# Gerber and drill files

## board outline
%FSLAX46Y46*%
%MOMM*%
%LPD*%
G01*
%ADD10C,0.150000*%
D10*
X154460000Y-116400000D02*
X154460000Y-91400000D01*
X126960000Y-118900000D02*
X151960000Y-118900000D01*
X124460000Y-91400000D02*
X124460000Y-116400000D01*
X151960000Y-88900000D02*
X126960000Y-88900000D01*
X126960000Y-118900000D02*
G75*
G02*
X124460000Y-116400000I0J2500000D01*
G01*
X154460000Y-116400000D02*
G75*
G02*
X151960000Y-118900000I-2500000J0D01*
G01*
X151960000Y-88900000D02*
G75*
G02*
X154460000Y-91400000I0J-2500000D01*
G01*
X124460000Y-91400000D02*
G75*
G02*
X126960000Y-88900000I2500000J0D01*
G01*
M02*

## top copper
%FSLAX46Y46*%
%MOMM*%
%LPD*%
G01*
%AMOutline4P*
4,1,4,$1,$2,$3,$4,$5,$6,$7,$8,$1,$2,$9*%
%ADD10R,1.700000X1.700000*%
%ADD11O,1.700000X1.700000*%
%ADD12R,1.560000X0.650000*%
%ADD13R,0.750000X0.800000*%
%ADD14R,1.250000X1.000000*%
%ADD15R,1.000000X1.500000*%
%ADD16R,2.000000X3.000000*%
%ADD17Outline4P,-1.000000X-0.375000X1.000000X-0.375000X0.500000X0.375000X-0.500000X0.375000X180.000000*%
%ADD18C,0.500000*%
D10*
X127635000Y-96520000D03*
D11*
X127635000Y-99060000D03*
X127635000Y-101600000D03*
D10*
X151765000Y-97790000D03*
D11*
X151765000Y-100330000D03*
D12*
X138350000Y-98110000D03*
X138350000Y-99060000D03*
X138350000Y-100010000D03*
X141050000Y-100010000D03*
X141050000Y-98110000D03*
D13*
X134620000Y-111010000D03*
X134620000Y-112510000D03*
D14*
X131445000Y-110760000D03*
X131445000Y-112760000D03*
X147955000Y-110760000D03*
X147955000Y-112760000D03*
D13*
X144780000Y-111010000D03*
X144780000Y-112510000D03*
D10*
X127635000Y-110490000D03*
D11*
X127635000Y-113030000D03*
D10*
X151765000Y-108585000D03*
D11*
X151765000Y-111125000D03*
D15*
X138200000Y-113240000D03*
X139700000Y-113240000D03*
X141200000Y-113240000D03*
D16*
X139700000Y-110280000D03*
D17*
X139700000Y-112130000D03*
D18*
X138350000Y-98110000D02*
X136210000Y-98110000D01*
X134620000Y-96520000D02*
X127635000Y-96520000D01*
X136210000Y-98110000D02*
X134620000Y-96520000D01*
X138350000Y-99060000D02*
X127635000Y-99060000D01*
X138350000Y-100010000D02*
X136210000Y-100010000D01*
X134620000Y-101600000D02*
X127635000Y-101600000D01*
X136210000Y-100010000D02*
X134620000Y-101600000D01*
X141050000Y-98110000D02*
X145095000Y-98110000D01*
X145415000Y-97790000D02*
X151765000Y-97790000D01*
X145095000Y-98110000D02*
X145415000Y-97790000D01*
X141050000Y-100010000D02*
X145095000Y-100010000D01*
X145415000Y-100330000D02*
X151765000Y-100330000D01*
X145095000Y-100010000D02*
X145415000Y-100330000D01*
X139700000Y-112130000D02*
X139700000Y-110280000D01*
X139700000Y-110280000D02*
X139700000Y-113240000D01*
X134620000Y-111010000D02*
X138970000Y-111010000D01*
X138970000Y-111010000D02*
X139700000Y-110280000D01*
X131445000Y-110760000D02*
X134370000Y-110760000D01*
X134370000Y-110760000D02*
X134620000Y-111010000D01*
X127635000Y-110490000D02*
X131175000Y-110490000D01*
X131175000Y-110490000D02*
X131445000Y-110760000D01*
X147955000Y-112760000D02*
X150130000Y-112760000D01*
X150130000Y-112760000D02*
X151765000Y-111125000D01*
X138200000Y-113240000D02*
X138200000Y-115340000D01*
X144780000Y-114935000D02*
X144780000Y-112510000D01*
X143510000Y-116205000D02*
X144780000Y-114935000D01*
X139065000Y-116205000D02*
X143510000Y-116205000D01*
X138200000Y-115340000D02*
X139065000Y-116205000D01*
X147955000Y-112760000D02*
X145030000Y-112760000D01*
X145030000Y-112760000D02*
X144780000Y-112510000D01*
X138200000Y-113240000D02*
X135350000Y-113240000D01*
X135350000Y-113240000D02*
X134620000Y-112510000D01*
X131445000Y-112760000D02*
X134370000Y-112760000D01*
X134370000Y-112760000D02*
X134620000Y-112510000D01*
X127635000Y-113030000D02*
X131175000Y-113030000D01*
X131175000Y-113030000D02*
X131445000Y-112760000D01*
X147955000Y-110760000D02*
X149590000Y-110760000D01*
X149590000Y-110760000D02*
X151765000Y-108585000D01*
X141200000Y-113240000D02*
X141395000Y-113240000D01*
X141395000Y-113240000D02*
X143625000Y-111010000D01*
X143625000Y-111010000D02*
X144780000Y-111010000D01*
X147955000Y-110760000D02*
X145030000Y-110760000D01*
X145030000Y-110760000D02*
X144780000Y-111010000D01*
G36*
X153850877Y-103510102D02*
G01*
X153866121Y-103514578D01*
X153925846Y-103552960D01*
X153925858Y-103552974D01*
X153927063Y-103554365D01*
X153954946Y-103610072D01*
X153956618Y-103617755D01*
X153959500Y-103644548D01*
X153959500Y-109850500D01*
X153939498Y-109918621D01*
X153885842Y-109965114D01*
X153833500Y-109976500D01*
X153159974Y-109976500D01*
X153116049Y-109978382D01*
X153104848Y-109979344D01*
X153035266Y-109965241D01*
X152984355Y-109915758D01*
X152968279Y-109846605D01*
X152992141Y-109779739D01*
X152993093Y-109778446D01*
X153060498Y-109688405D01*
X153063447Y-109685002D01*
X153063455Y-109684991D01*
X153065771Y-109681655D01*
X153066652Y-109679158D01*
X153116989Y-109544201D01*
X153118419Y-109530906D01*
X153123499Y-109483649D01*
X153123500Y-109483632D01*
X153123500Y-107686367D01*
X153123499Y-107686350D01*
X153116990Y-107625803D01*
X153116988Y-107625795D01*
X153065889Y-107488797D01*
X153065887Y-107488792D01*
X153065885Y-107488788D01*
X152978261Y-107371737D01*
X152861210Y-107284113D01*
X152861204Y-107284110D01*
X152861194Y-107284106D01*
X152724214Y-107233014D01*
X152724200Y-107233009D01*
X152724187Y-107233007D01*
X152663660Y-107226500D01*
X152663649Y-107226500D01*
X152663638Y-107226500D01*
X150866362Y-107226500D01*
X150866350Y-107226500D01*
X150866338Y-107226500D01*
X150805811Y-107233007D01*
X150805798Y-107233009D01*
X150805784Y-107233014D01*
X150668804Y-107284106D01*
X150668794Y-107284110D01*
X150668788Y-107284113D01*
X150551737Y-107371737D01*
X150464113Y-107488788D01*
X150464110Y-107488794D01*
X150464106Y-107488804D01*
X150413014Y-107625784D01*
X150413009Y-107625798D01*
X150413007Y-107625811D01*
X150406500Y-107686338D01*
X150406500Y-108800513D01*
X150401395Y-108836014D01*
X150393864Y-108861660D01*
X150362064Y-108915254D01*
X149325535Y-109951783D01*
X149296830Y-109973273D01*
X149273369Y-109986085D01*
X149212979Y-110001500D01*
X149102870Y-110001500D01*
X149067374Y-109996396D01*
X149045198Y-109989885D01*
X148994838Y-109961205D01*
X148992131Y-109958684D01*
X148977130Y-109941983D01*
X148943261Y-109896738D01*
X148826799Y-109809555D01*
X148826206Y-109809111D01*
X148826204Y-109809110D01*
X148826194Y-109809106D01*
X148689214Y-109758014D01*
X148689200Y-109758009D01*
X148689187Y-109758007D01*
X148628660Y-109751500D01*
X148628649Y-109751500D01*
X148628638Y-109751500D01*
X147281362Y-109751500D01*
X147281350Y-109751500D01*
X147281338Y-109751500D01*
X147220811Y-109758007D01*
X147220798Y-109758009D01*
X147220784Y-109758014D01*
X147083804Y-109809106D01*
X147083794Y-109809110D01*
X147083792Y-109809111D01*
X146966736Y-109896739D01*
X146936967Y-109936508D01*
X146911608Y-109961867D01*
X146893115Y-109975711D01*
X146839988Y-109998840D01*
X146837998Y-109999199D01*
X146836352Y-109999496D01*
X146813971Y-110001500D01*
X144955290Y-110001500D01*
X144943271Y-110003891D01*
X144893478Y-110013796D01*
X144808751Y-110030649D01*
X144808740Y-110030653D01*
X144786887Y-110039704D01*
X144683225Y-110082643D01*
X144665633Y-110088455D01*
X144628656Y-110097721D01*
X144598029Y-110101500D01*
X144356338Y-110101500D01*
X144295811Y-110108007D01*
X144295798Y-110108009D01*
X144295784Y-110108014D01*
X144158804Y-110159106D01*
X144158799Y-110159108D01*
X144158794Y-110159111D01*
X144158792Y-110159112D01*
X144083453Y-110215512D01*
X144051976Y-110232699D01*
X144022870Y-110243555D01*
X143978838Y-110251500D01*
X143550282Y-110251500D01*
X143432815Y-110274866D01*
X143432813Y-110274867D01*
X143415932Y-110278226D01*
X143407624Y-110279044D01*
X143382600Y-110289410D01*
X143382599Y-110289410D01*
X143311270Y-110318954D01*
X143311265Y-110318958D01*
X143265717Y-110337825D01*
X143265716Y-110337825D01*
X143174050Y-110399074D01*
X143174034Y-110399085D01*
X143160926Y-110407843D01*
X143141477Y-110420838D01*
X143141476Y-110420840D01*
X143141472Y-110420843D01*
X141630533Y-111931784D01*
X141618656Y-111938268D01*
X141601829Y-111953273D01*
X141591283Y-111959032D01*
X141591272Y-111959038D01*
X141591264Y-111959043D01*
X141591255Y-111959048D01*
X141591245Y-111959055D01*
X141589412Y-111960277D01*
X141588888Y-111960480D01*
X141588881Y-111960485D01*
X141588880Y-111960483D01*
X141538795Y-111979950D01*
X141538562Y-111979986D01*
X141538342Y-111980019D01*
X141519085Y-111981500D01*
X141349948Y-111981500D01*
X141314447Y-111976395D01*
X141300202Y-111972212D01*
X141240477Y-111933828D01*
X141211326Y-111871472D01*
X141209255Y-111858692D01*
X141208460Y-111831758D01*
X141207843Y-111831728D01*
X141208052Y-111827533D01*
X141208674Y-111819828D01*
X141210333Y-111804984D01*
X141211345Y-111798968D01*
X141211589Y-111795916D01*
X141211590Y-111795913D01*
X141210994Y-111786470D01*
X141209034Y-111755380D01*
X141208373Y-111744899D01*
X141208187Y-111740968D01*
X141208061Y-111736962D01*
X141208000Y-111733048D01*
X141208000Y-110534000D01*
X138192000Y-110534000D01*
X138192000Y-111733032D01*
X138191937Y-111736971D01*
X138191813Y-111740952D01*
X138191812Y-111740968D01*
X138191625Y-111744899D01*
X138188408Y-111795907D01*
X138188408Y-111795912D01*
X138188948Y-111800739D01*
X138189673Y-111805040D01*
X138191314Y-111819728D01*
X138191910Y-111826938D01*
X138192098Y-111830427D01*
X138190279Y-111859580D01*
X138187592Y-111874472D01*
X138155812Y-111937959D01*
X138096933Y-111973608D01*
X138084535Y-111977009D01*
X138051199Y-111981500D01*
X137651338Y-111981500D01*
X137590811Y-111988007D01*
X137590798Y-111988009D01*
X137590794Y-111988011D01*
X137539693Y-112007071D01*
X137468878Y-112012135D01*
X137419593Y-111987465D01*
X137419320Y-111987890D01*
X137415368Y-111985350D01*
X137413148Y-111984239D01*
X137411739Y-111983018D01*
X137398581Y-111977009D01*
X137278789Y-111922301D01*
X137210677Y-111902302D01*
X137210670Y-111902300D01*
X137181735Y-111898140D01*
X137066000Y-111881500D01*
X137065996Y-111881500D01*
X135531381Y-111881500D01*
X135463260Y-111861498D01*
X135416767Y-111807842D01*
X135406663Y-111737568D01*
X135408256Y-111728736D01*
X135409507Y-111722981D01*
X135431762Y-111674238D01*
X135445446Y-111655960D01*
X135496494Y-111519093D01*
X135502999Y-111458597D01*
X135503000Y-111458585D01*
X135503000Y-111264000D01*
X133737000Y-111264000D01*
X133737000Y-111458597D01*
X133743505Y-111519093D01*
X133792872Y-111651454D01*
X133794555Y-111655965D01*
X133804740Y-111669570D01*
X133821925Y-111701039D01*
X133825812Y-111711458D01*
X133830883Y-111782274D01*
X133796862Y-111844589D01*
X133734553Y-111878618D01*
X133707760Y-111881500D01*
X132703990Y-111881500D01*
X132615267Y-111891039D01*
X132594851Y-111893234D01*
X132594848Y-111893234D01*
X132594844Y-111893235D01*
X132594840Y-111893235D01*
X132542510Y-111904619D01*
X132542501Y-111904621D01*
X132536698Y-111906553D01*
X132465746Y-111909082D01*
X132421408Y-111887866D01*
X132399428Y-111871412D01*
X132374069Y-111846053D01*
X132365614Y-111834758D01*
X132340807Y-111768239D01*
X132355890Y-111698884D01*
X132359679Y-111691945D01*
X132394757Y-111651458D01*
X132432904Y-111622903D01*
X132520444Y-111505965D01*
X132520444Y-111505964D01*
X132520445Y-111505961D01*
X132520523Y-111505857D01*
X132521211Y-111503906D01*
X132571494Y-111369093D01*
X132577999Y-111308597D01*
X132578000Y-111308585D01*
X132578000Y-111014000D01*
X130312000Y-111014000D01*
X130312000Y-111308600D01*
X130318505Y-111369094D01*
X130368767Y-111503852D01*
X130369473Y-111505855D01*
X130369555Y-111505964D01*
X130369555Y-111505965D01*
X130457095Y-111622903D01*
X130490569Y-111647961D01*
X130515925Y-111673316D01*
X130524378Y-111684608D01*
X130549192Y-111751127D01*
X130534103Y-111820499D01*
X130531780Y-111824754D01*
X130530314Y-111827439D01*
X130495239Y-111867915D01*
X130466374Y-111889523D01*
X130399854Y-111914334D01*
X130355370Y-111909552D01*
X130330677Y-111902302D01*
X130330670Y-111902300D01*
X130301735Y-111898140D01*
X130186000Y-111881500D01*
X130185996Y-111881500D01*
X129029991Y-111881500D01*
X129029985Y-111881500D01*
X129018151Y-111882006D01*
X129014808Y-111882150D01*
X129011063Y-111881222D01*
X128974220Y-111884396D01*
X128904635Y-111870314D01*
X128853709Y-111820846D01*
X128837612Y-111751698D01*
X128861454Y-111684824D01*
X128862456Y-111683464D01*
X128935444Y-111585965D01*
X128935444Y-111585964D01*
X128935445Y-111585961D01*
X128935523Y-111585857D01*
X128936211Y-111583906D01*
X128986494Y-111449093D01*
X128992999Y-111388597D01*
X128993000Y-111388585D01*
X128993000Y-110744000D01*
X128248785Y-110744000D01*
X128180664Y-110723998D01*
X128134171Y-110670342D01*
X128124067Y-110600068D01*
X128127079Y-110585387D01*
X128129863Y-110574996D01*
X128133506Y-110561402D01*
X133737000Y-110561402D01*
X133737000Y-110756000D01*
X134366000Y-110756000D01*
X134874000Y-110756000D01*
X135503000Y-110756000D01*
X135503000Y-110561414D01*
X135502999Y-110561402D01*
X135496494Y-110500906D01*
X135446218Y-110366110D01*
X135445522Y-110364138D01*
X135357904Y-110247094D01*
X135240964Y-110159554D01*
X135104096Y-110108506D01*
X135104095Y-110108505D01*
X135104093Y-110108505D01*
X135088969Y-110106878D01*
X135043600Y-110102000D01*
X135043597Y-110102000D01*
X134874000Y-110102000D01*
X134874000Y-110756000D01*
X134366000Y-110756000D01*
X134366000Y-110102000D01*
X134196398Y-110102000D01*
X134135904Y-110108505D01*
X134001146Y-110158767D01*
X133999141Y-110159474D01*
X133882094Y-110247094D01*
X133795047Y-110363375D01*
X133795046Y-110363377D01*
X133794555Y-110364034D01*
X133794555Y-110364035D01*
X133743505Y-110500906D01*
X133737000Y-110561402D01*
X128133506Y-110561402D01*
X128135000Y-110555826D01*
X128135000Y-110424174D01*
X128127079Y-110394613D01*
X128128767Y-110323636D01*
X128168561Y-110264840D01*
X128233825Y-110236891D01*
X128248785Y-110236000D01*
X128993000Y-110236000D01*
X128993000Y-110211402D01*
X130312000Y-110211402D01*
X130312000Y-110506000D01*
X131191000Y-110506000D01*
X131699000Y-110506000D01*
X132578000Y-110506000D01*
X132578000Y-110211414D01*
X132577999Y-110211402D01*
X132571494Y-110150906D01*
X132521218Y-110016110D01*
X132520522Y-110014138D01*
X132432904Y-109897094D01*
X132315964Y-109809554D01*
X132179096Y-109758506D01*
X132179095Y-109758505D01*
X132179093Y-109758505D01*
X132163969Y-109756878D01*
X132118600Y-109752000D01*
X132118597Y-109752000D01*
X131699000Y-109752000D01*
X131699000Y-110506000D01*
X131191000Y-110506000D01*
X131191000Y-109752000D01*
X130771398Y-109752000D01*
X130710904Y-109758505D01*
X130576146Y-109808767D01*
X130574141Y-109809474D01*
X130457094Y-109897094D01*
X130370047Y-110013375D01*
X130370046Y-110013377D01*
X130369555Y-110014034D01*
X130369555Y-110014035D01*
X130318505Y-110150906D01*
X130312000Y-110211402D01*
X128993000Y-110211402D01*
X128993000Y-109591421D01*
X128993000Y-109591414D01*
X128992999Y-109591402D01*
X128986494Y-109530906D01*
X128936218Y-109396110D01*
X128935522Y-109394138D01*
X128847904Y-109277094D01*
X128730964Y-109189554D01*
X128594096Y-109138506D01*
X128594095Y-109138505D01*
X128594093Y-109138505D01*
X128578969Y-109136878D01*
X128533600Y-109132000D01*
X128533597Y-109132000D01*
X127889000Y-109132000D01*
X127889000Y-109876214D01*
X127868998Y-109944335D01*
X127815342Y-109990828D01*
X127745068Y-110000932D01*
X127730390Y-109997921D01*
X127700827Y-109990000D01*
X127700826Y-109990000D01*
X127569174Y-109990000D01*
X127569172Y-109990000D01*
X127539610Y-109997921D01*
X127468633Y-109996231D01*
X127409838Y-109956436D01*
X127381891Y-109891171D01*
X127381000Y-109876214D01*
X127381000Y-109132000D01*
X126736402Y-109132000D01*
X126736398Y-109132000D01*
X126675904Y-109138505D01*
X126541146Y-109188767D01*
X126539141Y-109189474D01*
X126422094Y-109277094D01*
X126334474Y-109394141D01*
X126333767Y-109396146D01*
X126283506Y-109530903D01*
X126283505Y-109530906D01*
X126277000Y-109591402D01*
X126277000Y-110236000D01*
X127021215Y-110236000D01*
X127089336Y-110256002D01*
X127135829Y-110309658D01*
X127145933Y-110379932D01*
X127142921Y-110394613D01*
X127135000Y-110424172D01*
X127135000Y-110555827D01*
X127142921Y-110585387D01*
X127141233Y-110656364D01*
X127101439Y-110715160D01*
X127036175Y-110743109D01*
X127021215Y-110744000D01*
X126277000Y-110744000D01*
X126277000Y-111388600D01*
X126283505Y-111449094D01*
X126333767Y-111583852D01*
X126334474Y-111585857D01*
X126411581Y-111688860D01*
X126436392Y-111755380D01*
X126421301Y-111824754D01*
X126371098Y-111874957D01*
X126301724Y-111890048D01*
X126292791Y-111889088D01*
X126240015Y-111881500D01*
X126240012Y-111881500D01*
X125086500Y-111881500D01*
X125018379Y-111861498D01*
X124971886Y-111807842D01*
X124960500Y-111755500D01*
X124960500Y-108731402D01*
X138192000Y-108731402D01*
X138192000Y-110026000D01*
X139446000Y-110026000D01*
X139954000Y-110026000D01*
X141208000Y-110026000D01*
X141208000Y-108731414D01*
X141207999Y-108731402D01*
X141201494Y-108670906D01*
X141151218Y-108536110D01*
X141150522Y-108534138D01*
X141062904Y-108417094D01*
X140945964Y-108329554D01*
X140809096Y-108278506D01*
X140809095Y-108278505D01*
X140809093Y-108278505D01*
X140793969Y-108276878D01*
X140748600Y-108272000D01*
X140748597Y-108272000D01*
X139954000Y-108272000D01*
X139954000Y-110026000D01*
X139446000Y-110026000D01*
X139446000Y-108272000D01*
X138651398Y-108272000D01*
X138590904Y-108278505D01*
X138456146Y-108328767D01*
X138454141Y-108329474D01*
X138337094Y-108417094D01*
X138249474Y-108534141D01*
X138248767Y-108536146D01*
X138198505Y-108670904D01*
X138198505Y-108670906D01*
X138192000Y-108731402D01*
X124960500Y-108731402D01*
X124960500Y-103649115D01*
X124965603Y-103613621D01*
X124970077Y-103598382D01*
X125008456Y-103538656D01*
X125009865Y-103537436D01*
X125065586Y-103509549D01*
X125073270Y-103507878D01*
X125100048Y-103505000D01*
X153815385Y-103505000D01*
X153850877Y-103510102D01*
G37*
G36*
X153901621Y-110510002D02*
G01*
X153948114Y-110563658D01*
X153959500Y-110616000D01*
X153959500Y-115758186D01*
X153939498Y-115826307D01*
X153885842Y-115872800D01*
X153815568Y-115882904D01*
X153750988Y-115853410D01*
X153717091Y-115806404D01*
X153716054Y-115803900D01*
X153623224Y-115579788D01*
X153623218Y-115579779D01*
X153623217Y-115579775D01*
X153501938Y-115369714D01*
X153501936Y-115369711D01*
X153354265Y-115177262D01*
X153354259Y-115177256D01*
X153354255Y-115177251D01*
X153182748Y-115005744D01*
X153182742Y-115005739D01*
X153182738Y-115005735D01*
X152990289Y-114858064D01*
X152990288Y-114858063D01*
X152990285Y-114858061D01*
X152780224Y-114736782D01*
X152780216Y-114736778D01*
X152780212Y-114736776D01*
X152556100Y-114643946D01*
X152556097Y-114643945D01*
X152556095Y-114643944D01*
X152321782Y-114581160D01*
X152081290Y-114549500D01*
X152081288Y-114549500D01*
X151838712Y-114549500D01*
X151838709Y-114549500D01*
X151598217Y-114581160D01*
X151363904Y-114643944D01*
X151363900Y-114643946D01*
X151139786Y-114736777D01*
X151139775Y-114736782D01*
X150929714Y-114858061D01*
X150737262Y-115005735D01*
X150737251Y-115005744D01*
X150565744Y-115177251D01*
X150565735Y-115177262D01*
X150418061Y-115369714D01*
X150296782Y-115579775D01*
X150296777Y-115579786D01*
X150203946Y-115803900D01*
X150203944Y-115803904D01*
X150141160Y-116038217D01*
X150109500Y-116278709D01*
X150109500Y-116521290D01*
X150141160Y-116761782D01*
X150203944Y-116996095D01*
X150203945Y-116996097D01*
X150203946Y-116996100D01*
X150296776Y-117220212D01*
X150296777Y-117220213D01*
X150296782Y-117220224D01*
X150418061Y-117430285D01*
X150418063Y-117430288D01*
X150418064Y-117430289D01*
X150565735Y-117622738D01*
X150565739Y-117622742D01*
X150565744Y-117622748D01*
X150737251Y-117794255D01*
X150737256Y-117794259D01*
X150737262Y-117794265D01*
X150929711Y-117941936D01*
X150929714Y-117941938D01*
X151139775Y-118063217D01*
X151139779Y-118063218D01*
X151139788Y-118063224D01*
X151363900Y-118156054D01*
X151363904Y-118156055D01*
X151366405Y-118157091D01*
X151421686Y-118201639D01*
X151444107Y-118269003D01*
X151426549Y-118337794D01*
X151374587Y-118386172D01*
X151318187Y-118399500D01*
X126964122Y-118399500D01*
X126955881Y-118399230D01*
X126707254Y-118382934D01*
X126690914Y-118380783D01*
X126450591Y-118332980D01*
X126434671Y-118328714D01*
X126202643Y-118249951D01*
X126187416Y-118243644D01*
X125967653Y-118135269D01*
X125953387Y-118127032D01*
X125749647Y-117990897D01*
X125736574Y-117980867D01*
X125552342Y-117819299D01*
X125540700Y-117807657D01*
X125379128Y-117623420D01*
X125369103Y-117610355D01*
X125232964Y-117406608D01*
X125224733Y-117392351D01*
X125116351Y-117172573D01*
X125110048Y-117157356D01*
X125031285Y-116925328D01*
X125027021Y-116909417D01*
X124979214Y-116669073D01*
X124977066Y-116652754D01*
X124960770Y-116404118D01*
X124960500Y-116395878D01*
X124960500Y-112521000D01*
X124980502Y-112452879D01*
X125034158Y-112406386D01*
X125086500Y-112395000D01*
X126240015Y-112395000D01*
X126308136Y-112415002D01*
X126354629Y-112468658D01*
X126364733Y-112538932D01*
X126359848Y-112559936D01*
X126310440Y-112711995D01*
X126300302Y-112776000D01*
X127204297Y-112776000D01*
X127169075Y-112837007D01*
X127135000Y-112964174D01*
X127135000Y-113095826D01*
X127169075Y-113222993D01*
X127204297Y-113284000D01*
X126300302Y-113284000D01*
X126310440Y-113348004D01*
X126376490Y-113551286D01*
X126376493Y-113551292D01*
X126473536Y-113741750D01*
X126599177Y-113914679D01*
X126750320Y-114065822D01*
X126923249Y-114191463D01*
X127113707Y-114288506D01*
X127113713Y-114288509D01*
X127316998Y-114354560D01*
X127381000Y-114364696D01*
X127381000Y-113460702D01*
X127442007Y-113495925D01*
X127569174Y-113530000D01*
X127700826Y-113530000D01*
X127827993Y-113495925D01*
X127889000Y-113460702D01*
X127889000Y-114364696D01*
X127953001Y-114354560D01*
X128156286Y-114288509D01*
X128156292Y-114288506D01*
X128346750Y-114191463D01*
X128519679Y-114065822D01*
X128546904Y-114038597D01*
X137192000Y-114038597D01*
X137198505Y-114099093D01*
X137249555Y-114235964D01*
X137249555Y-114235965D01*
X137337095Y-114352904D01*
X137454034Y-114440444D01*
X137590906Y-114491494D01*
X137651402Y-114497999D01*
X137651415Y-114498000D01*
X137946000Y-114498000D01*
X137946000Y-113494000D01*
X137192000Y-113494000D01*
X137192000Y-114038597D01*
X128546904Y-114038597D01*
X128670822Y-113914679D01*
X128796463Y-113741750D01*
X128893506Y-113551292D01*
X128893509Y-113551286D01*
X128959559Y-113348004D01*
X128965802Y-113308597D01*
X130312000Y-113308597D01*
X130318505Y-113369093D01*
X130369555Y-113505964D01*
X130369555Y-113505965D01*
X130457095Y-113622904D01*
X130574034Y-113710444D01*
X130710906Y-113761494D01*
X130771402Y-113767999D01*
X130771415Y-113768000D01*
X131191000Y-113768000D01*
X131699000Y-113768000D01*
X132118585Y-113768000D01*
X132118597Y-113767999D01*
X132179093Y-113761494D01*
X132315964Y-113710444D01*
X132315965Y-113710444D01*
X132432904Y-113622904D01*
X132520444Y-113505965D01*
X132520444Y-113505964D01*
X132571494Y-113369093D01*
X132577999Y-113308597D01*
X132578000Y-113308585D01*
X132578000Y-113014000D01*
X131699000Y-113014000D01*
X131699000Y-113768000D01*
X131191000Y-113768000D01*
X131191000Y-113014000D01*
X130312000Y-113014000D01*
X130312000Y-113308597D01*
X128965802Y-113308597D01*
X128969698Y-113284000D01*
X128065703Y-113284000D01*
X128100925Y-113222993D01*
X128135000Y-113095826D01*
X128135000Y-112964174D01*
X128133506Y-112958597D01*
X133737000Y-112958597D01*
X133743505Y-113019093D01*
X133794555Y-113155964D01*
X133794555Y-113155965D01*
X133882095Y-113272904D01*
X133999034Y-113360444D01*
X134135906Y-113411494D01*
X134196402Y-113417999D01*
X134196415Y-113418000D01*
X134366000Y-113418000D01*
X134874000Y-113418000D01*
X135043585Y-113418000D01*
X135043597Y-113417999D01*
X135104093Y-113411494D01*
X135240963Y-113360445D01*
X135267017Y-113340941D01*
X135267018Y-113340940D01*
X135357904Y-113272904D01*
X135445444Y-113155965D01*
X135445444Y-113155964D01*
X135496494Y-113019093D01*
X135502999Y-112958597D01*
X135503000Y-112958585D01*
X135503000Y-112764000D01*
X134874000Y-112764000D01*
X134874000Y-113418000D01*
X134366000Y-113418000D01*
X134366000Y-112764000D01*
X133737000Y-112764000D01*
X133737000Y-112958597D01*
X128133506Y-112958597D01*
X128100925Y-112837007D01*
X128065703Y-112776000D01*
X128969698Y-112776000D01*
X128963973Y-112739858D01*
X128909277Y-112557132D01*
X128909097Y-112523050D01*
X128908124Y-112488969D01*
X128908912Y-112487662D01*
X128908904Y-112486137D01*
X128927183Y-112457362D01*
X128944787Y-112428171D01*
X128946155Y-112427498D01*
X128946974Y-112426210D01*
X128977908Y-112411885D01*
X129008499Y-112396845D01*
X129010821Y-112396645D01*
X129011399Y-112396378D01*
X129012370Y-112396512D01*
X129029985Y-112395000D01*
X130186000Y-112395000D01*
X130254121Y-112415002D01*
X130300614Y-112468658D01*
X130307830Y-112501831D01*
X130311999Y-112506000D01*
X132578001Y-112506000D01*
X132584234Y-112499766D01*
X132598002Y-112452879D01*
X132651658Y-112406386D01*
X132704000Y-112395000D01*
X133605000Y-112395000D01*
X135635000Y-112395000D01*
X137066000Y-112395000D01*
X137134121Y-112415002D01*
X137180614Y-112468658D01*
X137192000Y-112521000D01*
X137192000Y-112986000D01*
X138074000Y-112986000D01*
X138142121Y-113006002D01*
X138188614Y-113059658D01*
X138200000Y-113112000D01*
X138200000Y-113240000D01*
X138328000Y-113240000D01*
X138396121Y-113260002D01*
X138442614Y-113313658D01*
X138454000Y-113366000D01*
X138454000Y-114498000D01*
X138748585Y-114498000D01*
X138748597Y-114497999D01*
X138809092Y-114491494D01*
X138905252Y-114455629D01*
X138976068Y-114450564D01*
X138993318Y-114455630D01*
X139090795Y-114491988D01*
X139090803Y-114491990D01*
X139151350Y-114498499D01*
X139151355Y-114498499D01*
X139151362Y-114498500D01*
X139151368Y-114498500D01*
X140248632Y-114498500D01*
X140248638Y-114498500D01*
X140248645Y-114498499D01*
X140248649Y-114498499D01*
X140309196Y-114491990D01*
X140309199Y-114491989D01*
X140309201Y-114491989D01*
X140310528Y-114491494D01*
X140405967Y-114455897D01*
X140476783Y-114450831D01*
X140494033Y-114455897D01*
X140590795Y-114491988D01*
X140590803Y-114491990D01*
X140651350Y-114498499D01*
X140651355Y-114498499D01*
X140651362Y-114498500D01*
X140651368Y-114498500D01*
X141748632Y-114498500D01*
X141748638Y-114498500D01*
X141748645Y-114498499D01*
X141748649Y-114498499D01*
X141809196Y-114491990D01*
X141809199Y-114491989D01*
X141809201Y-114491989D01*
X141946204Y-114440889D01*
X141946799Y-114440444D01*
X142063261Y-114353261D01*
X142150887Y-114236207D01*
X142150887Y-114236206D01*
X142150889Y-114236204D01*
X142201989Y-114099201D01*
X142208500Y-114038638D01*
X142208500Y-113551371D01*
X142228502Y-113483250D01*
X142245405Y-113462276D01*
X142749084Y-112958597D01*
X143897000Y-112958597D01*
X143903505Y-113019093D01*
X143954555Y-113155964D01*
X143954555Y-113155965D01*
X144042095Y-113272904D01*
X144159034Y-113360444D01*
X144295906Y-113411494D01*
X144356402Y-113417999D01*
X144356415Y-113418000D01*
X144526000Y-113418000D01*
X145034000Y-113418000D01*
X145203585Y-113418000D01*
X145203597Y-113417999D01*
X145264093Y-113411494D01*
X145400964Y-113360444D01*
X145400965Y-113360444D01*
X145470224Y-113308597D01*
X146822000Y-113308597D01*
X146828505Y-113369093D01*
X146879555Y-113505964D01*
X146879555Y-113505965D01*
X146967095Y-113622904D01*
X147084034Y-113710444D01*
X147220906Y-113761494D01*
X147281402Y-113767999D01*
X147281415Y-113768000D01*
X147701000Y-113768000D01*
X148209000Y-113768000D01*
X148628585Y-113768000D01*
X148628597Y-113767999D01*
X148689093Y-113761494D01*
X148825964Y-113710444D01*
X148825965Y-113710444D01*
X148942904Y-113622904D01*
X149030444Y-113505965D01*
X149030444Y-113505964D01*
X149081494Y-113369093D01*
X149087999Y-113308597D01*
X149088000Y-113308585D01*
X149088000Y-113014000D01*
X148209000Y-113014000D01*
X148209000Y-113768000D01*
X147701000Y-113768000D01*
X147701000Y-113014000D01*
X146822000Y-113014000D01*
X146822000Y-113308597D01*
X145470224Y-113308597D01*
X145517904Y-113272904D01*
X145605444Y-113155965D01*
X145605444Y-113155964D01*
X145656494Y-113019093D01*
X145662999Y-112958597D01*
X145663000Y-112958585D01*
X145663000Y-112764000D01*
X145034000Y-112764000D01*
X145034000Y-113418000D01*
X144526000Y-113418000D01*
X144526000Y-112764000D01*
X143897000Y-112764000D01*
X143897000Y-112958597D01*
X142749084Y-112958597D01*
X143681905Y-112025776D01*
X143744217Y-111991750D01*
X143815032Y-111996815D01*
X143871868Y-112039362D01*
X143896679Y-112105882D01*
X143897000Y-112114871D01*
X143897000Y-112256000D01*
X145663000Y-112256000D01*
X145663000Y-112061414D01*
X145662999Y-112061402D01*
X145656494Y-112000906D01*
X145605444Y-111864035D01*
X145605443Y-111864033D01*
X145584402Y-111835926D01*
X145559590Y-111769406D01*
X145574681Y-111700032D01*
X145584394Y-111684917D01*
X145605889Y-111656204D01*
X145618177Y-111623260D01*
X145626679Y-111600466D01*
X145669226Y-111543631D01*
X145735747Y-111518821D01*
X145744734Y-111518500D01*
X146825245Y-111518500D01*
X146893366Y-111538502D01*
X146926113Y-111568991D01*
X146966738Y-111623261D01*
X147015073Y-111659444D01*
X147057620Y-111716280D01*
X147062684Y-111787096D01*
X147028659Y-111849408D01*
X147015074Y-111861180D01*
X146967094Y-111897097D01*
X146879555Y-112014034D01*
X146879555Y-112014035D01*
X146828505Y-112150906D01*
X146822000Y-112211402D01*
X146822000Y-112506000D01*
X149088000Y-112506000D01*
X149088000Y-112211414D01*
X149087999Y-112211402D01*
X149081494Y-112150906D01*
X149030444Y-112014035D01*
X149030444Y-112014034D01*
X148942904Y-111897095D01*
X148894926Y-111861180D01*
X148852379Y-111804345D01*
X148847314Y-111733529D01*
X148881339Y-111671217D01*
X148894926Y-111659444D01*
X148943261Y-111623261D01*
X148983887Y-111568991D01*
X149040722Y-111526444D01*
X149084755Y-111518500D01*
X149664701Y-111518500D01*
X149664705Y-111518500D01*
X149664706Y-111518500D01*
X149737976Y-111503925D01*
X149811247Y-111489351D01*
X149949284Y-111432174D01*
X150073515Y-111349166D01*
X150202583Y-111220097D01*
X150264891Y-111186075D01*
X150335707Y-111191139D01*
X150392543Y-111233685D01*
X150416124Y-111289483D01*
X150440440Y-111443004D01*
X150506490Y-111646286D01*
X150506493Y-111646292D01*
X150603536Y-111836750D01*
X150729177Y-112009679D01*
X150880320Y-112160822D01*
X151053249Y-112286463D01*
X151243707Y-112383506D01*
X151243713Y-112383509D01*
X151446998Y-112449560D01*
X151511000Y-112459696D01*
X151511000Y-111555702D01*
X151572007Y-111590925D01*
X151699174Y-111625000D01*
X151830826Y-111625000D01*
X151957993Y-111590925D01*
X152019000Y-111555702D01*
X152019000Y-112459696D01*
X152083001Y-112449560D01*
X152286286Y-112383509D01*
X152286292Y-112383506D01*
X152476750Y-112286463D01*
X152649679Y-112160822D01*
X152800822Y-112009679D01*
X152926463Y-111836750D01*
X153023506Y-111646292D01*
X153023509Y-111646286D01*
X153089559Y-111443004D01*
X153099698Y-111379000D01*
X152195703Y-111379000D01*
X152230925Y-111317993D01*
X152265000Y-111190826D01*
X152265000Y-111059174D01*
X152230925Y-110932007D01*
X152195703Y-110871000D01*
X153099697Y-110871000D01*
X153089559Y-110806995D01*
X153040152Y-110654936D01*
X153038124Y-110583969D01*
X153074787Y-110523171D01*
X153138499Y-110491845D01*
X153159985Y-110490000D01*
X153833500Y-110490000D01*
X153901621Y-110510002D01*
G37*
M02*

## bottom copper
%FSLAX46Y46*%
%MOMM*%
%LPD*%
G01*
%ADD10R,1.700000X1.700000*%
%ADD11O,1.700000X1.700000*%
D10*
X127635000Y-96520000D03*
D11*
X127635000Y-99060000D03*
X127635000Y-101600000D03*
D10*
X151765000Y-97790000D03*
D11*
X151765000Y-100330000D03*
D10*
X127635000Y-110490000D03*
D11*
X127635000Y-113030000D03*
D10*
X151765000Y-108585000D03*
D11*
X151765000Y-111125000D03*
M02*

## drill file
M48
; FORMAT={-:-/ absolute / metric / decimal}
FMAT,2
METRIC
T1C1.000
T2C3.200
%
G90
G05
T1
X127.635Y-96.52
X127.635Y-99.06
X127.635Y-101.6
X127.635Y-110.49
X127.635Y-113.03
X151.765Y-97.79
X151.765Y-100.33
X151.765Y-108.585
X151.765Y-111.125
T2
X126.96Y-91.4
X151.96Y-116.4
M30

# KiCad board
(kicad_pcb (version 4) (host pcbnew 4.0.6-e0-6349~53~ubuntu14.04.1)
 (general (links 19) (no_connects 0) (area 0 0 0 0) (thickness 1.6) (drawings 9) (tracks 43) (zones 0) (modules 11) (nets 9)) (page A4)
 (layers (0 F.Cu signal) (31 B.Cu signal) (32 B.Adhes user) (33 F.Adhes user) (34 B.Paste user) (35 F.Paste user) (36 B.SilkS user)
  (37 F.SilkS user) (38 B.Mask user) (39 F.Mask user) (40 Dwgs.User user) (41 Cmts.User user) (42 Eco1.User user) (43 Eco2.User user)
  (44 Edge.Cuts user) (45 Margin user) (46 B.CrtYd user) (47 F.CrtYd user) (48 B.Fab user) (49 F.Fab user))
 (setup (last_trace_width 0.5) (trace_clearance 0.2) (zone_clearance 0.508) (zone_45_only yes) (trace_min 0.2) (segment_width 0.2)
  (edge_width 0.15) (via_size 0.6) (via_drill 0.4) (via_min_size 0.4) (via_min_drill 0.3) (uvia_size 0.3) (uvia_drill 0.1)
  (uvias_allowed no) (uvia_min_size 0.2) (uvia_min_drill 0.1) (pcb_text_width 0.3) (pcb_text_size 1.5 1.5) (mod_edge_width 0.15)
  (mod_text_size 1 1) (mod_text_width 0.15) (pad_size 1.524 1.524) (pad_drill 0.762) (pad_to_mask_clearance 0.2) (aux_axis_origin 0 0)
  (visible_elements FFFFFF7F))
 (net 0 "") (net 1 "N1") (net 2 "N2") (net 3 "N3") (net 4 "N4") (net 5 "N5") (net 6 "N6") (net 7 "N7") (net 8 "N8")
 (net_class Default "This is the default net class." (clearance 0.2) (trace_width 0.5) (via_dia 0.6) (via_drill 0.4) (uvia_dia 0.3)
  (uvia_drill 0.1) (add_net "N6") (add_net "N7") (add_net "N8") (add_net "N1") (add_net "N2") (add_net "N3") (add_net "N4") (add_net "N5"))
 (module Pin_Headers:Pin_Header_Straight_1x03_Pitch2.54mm (layer F.Cu) (at 127.635 96.52)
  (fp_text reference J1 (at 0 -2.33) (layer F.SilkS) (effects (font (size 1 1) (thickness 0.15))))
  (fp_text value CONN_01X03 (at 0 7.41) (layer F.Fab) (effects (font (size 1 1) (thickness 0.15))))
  (pad 1 thru_hole rect (at 0 0) (size 1.7 1.7) (drill 1) (layers *.Cu *.Mask) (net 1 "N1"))
  (pad 2 thru_hole oval (at 0 2.54) (size 1.7 1.7) (drill 1) (layers *.Cu *.Mask) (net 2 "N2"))
  (pad 3 thru_hole oval (at 0 5.08) (size 1.7 1.7) (drill 1) (layers *.Cu *.Mask) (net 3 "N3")))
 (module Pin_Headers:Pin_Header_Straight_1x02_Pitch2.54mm (layer F.Cu) (at 151.765 97.79)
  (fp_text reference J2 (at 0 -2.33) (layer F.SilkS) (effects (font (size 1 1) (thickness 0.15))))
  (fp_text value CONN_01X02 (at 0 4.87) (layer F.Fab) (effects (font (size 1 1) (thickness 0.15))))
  (pad 1 thru_hole rect (at 0 0) (size 1.7 1.7) (drill 1) (layers *.Cu *.Mask) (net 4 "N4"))
  (pad 2 thru_hole oval (at 0 2.54) (size 1.7 1.7) (drill 1) (layers *.Cu *.Mask) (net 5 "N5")))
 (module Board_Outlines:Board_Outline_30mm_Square (layer F.Cu) (at 124.46 88.9)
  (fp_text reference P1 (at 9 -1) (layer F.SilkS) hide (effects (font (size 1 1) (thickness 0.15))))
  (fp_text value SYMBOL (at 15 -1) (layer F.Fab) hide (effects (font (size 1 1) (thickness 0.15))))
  (fp_line (start 30 27.5) (end 30 2.5) (layer Edge.Cuts) (width 0.15))
  (fp_line (start 2.5 30) (end 27.5 30) (layer Edge.Cuts) (width 0.15))
  (fp_line (start 0 2.5) (end 0 27.5) (layer Edge.Cuts) (width 0.15))
  (fp_line (start 27.5 0) (end 2.5 0) (layer Edge.Cuts) (width 0.15))
  (fp_arc (start 2.5 27.5) (end 2.5 30) (angle 90) (layer Edge.Cuts) (width 0.15))
  (fp_arc (start 27.5 27.5) (end 30 27.5) (angle 90) (layer Edge.Cuts) (width 0.15))
  (fp_arc (start 27.5 2.5) (end 27.5 0) (angle 90) (layer Edge.Cuts) (width 0.15))
  (fp_arc (start 2.5 2.5) (end 0 2.5) (angle 90) (layer Edge.Cuts) (width 0.15))
  (pad "" np_thru_hole circle (at 2.5 2.5) (size 3.2 3.2) (drill 3.2) (layers *.Cu *.Mask))
  (pad "" np_thru_hole circle (at 27.5 27.5) (size 3.2 3.2) (drill 3.2) (layers *.Cu *.Mask)))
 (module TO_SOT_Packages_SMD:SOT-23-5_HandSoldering (layer F.Cu) (at 139.7 99.06)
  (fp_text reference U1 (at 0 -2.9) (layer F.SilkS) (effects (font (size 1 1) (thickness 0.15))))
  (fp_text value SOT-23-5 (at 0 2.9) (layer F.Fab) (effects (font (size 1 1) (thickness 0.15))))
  (pad 1 smd rect (at -1.35 -0.95) (size 1.56 0.65) (layers F.Cu F.Paste F.Mask) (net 1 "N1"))
  (pad 2 smd rect (at -1.35 0) (size 1.56 0.65) (layers F.Cu F.Paste F.Mask) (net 2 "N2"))
  (pad 3 smd rect (at -1.35 0.95) (size 1.56 0.65) (layers F.Cu F.Paste F.Mask) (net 3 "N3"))
  (pad 4 smd rect (at 1.35 0.95) (size 1.56 0.65) (layers F.Cu F.Paste F.Mask) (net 5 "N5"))
  (pad 5 smd rect (at 1.35 -0.95) (size 1.56 0.65) (layers F.Cu F.Paste F.Mask) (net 4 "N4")))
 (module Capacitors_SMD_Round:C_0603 (layer F.Cu) (at 134.62 111.76 270)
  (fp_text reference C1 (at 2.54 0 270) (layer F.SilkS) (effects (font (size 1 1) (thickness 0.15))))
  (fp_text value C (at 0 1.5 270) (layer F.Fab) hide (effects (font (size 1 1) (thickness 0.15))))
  (pad 1 smd rect (at -0.75 0 270) (size 0.8 0.75) (layers F.Cu F.Paste F.Mask) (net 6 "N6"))
  (pad 2 smd rect (at 0.75 0 270) (size 0.8 0.75) (layers F.Cu F.Paste F.Mask) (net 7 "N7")))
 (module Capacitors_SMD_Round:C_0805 (layer F.Cu) (at 131.445 111.76 270)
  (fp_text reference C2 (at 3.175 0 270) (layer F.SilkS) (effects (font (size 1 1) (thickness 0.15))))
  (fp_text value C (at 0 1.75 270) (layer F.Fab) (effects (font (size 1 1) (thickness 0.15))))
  (pad 1 smd rect (at -1 0 270) (size 1 1.25) (layers F.Cu F.Paste F.Mask) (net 6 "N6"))
  (pad 2 smd rect (at 1 0 270) (size 1 1.25) (layers F.Cu F.Paste F.Mask) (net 7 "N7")))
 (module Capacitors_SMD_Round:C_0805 (layer F.Cu) (at 147.955 111.76 270)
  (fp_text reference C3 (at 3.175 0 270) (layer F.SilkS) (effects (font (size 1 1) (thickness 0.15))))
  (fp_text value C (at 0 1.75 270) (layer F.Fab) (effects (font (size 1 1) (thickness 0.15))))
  (pad 1 smd rect (at -1 0 270) (size 1 1.25) (layers F.Cu F.Paste F.Mask) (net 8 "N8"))
  (pad 2 smd rect (at 1 0 270) (size 1 1.25) (layers F.Cu F.Paste F.Mask) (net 7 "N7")))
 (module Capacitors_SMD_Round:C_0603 (layer F.Cu) (at 144.78 111.76 270)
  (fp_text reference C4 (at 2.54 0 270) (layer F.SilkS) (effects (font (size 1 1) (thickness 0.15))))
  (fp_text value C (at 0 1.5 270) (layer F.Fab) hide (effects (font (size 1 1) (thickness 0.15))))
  (pad 1 smd rect (at -0.75 0 270) (size 0.8 0.75) (layers F.Cu F.Paste F.Mask) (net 8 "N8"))
  (pad 2 smd rect (at 0.75 0 270) (size 0.8 0.75) (layers F.Cu F.Paste F.Mask) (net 7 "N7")))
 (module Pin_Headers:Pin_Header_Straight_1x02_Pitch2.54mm (layer F.Cu) (at 127.635 110.49)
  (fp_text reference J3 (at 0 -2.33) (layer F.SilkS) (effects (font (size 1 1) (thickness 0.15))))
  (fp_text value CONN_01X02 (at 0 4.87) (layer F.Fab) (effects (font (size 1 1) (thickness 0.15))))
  (pad 1 thru_hole rect (at 0 0) (size 1.7 1.7) (drill 1) (layers *.Cu *.Mask) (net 6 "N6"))
  (pad 2 thru_hole oval (at 0 2.54) (size 1.7 1.7) (drill 1) (layers *.Cu *.Mask) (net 7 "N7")))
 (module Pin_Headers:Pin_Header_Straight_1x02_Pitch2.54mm (layer F.Cu) (at 151.765 108.585)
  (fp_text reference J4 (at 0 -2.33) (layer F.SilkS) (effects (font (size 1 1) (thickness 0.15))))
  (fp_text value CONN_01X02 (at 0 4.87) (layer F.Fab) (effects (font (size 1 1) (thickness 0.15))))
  (pad 1 thru_hole rect (at 0 0) (size 1.7 1.7) (drill 1) (layers *.Cu *.Mask) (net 8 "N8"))
  (pad 2 thru_hole oval (at 0 2.54) (size 1.7 1.7) (drill 1) (layers *.Cu *.Mask) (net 7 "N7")))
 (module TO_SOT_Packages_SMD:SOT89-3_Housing (layer F.Cu) (at 139.7 111.76 90)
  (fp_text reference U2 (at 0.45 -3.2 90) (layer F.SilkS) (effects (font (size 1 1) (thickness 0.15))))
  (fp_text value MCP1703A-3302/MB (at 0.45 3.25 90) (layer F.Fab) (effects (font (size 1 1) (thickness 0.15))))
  (pad 1 smd rect (at -1.48 -1.5) (size 1 1.5) (layers F.Cu F.Paste F.Mask) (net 7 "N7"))
  (pad 2 smd rect (at -1.48 0) (size 1 1.5) (layers F.Cu F.Paste F.Mask) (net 6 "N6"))
  (pad 3 smd rect (at -1.48 1.5) (size 1 1.5) (layers F.Cu F.Paste F.Mask) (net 8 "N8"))
  (pad 2 smd rect (at 1.48 0) (size 2 3) (layers F.Cu F.Paste F.Mask) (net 6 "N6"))
  (pad 2 smd trapezoid (at -0.37 0 180) (size 1.5 0.75) (rect_delta 0 0.5) (layers F.Cu F.Paste F.Mask) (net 6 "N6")))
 (segment (start 138.35 98.11) (end 136.21 98.11) (width 0.5) (layer F.Cu) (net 1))
 (segment (start 134.62 96.52) (end 127.635 96.52) (width 0.5) (layer F.Cu) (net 1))
 (segment (start 136.21 98.11) (end 134.62 96.52) (width 0.5) (layer F.Cu) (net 1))
 (segment (start 138.35 99.06) (end 127.635 99.06) (width 0.5) (layer F.Cu) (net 2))
 (segment (start 138.35 100.01) (end 136.21 100.01) (width 0.5) (layer F.Cu) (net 3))
 (segment (start 134.62 101.6) (end 127.635 101.6) (width 0.5) (layer F.Cu) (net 3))
 (segment (start 136.21 100.01) (end 134.62 101.6) (width 0.5) (layer F.Cu) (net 3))
 (segment (start 141.05 98.11) (end 145.095 98.11) (width 0.5) (layer F.Cu) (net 4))
 (segment (start 145.415 97.79) (end 151.765 97.79) (width 0.5) (layer F.Cu) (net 4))
 (segment (start 145.095 98.11) (end 145.415 97.79) (width 0.5) (layer F.Cu) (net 4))
 (segment (start 141.05 100.01) (end 145.095 100.01) (width 0.5) (layer F.Cu) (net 5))
 (segment (start 145.415 100.33) (end 151.765 100.33) (width 0.5) (layer F.Cu) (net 5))
 (segment (start 145.095 100.01) (end 145.415 100.33) (width 0.5) (layer F.Cu) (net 5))
 (segment (start 139.7 112.13) (end 139.7 110.28) (width 0.5) (layer F.Cu) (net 6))
 (segment (start 139.7 110.28) (end 139.7 113.24) (width 0.5) (layer F.Cu) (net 6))
 (segment (start 134.62 111.01) (end 138.97 111.01) (width 0.5) (layer F.Cu) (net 6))
 (segment (start 138.97 111.01) (end 139.7 110.28) (width 0.5) (layer F.Cu) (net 6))
 (segment (start 131.445 110.76) (end 134.37 110.76) (width 0.5) (layer F.Cu) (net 6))
 (segment (start 134.37 110.76) (end 134.62 111.01) (width 0.5) (layer F.Cu) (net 6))
 (segment (start 127.635 110.49) (end 131.175 110.49) (width 0.5) (layer F.Cu) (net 6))
 (segment (start 131.175 110.49) (end 131.445 110.76) (width 0.5) (layer F.Cu) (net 6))
 (segment (start 147.955 112.76) (end 150.13 112.76) (width 0.5) (layer F.Cu) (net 7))
 (segment (start 150.13 112.76) (end 151.765 111.125) (width 0.5) (layer F.Cu) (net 7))
 (segment (start 138.2 113.24) (end 138.2 115.34) (width 0.5) (layer F.Cu) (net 7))
 (segment (start 144.78 114.935) (end 144.78 112.51) (width 0.5) (layer F.Cu) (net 7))
 (segment (start 143.51 116.205) (end 144.78 114.935) (width 0.5) (layer F.Cu) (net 7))
 (segment (start 139.065 116.205) (end 143.51 116.205) (width 0.5) (layer F.Cu) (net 7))
 (segment (start 138.2 115.34) (end 139.065 116.205) (width 0.5) (layer F.Cu) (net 7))
 (segment (start 147.955 112.76) (end 145.03 112.76) (width 0.5) (layer F.Cu) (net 7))
 (segment (start 145.03 112.76) (end 144.78 112.51) (width 0.5) (layer F.Cu) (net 7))
 (segment (start 138.2 113.24) (end 135.35 113.24) (width 0.5) (layer F.Cu) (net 7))
 (segment (start 135.35 113.24) (end 134.62 112.51) (width 0.5) (layer F.Cu) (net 7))
 (segment (start 131.445 112.76) (end 134.37 112.76) (width 0.5) (layer F.Cu) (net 7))
 (segment (start 134.37 112.76) (end 134.62 112.51) (width 0.5) (layer F.Cu) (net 7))
 (segment (start 127.635 113.03) (end 131.175 113.03) (width 0.5) (layer F.Cu) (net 7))
 (segment (start 131.175 113.03) (end 131.445 112.76) (width 0.5) (layer F.Cu) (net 7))
 (segment (start 147.955 110.76) (end 149.59 110.76) (width 0.5) (layer F.Cu) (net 8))
 (segment (start 149.59 110.76) (end 151.765 108.585) (width 0.5) (layer F.Cu) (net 8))
 (segment (start 141.2 113.24) (end 141.395 113.24) (width 0.5) (layer F.Cu) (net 8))
 (segment (start 141.395 113.24) (end 143.625 111.01) (width 0.5) (layer F.Cu) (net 8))
 (segment (start 143.625 111.01) (end 144.78 111.01) (width 0.5) (layer F.Cu) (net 8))
 (segment (start 147.955 110.76) (end 145.03 110.76) (width 0.5) (layer F.Cu) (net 8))
 (segment (start 145.03 110.76) (end 144.78 111.01) (width 0.5) (layer F.Cu) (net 8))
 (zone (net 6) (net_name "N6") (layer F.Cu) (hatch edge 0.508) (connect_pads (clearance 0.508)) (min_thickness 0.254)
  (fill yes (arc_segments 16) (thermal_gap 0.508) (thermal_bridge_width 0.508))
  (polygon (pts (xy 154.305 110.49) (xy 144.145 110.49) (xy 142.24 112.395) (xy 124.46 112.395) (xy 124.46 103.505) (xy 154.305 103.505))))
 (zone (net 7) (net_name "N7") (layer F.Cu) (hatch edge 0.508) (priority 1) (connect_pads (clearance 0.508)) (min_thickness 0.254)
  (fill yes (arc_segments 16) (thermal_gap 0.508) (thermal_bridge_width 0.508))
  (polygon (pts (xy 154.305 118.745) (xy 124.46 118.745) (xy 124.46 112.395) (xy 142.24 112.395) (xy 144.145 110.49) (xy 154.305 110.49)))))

